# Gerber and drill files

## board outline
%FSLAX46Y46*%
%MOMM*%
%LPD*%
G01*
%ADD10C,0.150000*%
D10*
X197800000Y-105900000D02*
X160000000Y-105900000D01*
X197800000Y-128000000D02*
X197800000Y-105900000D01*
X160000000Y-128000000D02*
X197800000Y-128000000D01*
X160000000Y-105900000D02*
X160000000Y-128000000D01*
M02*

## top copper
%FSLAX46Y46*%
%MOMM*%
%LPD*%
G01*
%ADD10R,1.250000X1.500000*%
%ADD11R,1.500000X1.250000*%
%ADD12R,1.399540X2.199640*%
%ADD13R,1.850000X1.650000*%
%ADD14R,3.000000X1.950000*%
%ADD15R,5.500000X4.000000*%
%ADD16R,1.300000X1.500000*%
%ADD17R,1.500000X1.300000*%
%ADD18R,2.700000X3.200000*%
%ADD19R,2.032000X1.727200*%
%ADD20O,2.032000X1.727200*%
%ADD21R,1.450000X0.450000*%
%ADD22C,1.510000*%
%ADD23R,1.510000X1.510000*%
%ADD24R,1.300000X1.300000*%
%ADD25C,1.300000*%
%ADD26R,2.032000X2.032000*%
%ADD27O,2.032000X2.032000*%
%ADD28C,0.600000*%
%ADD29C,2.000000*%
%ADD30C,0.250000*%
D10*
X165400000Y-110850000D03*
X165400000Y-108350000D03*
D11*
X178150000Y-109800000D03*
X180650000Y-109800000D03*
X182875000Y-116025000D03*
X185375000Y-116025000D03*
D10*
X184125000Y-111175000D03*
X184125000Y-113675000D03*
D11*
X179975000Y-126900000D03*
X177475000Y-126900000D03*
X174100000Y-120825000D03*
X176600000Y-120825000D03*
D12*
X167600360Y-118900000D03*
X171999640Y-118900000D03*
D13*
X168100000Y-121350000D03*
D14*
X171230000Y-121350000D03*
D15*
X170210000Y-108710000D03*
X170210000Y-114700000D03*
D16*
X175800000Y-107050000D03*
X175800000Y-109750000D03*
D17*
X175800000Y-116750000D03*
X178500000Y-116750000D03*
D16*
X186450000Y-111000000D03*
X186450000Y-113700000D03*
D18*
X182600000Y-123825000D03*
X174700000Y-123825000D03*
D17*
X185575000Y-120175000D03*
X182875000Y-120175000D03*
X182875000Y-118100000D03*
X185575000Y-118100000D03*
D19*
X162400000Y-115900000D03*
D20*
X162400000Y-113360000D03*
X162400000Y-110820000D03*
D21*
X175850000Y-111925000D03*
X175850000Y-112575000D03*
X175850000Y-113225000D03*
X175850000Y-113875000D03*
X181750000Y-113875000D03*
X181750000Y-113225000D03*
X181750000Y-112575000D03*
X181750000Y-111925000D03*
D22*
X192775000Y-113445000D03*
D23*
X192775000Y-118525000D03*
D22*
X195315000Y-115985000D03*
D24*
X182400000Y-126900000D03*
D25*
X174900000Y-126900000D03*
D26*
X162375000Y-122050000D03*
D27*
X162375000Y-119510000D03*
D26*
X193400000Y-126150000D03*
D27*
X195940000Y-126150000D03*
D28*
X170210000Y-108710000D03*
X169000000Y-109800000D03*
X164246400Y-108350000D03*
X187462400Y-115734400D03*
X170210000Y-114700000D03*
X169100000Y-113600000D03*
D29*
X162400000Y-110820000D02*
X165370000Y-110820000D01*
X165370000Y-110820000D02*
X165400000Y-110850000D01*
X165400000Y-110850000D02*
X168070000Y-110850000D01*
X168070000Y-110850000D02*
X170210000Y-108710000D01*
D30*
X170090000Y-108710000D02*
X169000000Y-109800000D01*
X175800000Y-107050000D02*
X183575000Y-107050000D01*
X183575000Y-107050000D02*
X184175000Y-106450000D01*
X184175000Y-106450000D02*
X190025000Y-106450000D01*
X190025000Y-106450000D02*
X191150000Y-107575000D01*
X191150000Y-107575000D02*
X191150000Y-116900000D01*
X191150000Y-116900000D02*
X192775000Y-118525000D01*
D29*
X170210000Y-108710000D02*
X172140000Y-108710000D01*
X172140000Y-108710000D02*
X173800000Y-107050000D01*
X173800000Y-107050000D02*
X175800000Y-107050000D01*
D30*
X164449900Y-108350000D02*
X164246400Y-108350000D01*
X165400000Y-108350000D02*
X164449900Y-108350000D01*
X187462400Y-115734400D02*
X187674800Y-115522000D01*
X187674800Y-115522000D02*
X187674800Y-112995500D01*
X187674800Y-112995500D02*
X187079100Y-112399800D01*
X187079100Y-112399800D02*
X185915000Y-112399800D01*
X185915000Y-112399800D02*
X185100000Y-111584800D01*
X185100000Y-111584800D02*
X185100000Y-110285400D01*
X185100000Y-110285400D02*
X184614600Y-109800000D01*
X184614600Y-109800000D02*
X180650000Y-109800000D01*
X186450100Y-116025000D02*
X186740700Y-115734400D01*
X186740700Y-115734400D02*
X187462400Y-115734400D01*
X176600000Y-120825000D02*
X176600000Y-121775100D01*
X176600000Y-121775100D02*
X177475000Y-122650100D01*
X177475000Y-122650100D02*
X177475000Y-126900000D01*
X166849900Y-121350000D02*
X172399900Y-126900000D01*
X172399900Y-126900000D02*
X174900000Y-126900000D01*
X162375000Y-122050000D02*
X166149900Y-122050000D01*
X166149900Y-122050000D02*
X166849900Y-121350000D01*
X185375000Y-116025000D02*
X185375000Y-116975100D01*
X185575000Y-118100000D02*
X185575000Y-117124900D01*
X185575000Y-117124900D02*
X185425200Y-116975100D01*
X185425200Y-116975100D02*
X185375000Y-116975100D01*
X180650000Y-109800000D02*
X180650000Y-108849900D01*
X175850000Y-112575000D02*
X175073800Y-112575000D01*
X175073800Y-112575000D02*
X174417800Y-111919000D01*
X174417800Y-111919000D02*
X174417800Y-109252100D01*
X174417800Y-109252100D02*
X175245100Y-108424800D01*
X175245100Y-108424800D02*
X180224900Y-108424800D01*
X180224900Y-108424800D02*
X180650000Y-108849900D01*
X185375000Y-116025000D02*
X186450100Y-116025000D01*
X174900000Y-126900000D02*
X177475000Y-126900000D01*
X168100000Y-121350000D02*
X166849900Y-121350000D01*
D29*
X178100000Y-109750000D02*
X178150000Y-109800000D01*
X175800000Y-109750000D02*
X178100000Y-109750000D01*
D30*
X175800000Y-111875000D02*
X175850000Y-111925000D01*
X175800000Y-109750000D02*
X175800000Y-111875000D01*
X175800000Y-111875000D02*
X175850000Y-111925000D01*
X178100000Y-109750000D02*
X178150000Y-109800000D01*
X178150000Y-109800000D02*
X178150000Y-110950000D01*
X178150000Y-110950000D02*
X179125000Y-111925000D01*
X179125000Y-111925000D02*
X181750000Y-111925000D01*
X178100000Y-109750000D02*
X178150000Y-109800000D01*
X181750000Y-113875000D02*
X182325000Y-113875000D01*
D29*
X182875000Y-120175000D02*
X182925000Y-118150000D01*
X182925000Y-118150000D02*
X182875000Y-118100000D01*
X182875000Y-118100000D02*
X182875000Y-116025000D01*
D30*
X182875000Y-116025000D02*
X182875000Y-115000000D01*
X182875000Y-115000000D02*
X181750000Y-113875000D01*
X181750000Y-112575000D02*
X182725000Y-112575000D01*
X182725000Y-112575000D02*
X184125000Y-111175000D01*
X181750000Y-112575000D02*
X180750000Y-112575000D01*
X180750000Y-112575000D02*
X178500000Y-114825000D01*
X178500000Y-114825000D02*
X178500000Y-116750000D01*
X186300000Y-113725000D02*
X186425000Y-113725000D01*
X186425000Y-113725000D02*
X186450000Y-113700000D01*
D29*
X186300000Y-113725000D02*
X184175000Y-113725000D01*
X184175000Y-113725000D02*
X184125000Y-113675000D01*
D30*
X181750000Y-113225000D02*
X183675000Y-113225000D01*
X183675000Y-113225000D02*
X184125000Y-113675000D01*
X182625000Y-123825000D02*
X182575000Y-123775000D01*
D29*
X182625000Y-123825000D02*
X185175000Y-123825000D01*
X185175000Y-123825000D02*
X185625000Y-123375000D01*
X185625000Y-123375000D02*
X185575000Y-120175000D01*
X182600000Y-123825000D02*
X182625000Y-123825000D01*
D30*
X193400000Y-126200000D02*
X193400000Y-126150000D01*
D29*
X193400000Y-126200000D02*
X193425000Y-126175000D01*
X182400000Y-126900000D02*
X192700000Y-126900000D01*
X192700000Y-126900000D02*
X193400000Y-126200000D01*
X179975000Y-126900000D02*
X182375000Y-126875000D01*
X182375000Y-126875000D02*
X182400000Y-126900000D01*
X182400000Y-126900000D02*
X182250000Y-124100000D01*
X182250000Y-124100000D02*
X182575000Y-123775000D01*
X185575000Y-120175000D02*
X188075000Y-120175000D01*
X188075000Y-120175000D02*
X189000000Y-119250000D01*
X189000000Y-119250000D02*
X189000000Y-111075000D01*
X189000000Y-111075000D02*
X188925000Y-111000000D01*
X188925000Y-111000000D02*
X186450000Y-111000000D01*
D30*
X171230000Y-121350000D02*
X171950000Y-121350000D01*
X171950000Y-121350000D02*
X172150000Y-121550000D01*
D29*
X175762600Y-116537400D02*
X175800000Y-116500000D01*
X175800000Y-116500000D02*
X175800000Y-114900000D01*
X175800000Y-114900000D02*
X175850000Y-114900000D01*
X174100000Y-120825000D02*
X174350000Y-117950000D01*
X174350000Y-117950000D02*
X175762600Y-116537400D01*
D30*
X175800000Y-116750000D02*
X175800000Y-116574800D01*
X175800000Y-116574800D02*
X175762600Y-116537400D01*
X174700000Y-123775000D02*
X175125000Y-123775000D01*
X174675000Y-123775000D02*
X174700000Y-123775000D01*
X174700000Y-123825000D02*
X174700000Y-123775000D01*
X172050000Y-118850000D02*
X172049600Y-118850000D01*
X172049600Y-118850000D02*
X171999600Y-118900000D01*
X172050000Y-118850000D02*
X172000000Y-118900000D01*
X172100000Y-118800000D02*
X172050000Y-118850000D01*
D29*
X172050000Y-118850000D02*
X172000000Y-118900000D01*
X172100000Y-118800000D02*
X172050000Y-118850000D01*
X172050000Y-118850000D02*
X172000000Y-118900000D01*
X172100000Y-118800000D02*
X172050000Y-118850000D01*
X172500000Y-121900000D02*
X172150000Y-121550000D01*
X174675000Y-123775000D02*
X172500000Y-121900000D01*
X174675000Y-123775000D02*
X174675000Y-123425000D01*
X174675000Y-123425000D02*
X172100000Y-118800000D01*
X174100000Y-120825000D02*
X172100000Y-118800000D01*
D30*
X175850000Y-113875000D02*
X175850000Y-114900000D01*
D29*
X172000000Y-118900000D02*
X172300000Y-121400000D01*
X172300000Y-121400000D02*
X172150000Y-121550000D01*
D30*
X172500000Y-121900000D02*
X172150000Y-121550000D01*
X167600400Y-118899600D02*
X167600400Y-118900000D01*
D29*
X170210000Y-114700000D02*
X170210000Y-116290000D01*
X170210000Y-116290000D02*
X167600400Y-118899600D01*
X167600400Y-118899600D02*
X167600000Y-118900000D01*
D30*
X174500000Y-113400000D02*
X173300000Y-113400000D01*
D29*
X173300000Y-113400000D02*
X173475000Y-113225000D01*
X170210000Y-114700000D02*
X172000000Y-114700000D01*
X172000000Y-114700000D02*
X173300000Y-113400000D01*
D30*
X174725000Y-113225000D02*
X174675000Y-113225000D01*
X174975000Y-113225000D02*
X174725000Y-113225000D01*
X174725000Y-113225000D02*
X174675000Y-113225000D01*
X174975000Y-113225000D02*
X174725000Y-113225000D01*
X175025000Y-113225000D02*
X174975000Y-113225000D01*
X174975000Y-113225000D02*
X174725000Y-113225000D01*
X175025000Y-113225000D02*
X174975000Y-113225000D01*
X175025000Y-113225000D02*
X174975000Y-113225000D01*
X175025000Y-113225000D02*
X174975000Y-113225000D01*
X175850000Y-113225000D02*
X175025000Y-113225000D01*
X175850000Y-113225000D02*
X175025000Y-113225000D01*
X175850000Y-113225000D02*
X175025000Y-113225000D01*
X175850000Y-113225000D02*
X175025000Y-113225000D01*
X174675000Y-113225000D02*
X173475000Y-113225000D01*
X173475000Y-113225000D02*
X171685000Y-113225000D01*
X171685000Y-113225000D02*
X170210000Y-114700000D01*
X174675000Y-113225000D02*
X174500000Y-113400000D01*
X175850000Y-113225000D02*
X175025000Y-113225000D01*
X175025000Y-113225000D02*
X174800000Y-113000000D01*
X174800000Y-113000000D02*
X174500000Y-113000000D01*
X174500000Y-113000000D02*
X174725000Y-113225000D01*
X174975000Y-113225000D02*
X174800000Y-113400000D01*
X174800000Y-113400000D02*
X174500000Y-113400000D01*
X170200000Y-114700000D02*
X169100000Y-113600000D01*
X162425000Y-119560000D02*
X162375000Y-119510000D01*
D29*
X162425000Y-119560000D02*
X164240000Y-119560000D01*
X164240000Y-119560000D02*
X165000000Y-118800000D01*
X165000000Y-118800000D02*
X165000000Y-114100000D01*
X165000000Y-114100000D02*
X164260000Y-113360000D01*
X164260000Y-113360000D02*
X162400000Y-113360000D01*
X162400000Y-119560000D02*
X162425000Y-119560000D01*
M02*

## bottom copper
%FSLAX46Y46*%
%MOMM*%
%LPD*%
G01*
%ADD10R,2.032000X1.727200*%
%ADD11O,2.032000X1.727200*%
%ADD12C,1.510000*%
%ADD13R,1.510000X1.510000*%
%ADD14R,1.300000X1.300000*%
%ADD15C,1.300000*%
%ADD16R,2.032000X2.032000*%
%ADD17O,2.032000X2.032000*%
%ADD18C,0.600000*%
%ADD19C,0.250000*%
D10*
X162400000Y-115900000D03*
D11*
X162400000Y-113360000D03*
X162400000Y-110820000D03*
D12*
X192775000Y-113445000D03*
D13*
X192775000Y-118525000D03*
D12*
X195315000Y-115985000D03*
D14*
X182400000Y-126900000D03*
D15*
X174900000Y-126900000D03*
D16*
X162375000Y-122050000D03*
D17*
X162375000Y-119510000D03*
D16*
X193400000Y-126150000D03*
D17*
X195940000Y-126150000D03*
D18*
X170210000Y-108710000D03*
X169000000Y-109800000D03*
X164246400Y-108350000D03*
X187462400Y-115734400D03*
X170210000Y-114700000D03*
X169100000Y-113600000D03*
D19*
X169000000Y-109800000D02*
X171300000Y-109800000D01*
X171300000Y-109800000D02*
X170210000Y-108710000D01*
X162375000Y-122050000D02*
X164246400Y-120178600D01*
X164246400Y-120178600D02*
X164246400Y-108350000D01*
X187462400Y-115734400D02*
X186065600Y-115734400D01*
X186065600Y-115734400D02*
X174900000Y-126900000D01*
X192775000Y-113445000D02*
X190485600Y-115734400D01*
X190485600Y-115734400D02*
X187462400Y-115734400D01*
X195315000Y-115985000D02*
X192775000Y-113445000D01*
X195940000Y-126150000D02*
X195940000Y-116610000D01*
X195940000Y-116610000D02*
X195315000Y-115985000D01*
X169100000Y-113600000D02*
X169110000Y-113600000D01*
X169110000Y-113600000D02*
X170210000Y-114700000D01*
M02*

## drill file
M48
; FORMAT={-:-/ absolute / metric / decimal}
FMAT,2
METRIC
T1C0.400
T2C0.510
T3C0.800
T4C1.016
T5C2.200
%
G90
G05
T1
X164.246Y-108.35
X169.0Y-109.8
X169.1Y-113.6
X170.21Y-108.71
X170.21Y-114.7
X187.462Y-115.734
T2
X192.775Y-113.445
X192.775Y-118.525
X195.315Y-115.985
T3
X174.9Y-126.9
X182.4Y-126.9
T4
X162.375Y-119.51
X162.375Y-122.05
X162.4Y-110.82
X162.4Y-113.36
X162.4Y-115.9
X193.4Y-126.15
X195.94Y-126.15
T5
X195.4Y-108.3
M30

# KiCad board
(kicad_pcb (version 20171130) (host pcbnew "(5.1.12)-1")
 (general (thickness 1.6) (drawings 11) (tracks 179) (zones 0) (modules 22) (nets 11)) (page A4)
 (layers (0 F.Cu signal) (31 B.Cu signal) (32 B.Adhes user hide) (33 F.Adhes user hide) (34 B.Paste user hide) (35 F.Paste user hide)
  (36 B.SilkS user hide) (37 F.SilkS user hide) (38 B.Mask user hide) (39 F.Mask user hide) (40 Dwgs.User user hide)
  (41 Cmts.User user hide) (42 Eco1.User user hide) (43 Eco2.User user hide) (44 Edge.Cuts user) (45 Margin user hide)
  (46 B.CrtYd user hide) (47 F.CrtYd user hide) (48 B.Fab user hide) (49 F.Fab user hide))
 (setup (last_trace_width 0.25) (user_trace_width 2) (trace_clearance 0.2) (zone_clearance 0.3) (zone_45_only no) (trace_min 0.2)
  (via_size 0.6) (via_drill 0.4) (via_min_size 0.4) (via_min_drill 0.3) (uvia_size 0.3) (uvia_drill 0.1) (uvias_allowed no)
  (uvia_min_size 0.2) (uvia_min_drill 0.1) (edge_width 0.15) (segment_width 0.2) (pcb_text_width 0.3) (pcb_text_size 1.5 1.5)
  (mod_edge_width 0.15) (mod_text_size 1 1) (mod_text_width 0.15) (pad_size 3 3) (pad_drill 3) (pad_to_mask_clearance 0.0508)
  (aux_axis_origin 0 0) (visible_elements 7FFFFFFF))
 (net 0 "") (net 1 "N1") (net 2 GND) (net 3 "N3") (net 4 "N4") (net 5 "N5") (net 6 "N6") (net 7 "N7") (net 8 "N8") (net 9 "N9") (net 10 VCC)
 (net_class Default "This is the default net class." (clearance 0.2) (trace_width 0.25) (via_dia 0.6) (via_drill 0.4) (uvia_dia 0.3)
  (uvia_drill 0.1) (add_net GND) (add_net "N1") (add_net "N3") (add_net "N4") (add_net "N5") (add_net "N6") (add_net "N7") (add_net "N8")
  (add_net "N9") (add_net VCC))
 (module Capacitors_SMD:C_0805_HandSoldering (layer F.Cu) (at 165.4 109.6 90)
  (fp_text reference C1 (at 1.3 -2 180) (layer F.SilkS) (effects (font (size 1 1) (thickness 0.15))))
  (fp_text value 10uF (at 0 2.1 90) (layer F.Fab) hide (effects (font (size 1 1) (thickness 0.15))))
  (pad 1 smd rect (at -1.25 0 90) (size 1.5 1.25) (layers F.Cu F.Paste F.Mask) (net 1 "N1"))
  (pad 2 smd rect (at 1.25 0 90) (size 1.5 1.25) (layers F.Cu F.Paste F.Mask) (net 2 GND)))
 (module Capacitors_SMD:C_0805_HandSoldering (layer F.Cu) (at 179.4 109.8)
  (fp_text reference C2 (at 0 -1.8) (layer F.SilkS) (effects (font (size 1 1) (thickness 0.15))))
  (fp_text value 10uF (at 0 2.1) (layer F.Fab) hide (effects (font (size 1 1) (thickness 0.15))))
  (pad 1 smd rect (at -1.25 0) (size 1.5 1.25) (layers F.Cu F.Paste F.Mask) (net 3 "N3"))
  (pad 2 smd rect (at 1.25 0) (size 1.5 1.25) (layers F.Cu F.Paste F.Mask) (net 2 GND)))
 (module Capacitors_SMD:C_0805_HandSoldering (layer F.Cu) (at 184.125 116.025)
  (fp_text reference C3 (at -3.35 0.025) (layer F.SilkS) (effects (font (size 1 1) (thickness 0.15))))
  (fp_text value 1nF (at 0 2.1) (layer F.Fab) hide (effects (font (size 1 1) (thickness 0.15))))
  (pad 1 smd rect (at -1.25 0) (size 1.5 1.25) (layers F.Cu F.Paste F.Mask) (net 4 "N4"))
  (pad 2 smd rect (at 1.25 0) (size 1.5 1.25) (layers F.Cu F.Paste F.Mask) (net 2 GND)))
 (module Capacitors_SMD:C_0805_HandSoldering (layer F.Cu) (at 184.125 112.425 270)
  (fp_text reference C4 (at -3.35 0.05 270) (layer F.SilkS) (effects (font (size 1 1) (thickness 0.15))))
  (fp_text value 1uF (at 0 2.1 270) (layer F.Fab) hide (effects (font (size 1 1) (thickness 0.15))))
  (pad 1 smd rect (at -1.25 0 270) (size 1.5 1.25) (layers F.Cu F.Paste F.Mask) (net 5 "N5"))
  (pad 2 smd rect (at 1.25 0 270) (size 1.5 1.25) (layers F.Cu F.Paste F.Mask) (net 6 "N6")))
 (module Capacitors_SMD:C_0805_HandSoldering (layer F.Cu) (at 178.725 126.9 180)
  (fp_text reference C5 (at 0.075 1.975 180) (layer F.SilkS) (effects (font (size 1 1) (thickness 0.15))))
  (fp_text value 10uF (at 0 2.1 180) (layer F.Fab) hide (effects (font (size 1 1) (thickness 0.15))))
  (pad 1 smd rect (at -1.25 0 180) (size 1.5 1.25) (layers F.Cu F.Paste F.Mask) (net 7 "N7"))
  (pad 2 smd rect (at 1.25 0 180) (size 1.5 1.25) (layers F.Cu F.Paste F.Mask) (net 2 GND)))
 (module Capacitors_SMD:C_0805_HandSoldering (layer F.Cu) (at 175.35 120.825)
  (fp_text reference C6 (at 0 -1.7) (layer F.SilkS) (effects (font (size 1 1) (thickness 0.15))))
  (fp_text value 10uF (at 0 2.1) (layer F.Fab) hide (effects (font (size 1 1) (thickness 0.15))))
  (pad 1 smd rect (at -1.25 0) (size 1.5 1.25) (layers F.Cu F.Paste F.Mask) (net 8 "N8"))
  (pad 2 smd rect (at 1.25 0) (size 1.5 1.25) (layers F.Cu F.Paste F.Mask) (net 2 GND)))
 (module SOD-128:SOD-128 (layer F.Cu) (at 169.8 118.9)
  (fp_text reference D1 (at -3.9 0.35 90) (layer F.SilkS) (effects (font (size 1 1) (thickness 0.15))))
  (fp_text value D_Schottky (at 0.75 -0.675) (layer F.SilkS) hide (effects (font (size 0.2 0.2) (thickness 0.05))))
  (pad 2 smd rect (at -2.19964 0) (size 1.39954 2.19964) (layers F.Cu F.Paste F.Mask) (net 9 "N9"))
  (pad 1 smd rect (at 2.19964 0) (size 1.39954 2.19964) (layers F.Cu F.Paste F.Mask) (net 8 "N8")))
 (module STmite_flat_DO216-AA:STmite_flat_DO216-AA (layer F.Cu) (at 168.55 120.4)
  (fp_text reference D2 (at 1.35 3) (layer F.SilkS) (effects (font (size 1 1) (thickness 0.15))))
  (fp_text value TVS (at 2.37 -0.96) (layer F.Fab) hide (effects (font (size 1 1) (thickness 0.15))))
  (pad 1 smd rect (at -0.45 0.95) (size 1.85 1.65) (layers F.Cu F.Paste F.Mask) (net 2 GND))
  (pad 2 smd rect (at 2.68 0.95) (size 3 1.95) (layers F.Cu F.Paste F.Mask) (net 8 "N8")))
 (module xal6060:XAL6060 (layer F.Cu) (at 166.9 114.9 90)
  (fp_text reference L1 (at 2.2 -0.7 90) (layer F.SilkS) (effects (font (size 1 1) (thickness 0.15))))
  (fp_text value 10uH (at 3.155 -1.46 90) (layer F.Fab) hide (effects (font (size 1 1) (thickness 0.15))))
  (pad 2 smd rect (at 6.19 3.31 90) (size 4 5.5) (layers F.Cu F.Paste F.Mask) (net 1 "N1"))
  (pad 1 smd rect (at 0.2 3.31 90) (size 4 5.5) (layers F.Cu F.Paste F.Mask) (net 9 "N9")))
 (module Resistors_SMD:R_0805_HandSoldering (layer F.Cu) (at 175.8 108.4 270)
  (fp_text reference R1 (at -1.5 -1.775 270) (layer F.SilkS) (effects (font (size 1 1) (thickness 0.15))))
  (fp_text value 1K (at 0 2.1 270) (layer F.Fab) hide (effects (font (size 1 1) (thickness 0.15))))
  (pad 1 smd rect (at -1.35 0 270) (size 1.5 1.3) (layers F.Cu F.Paste F.Mask) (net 1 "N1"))
  (pad 2 smd rect (at 1.35 0 270) (size 1.5 1.3) (layers F.Cu F.Paste F.Mask) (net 3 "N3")))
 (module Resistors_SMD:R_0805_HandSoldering (layer F.Cu) (at 177.15 116.75)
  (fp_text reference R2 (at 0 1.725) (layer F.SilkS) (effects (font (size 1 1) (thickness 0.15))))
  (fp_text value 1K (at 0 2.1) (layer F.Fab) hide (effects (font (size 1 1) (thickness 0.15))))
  (pad 1 smd rect (at -1.35 0) (size 1.5 1.3) (layers F.Cu F.Paste F.Mask) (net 8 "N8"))
  (pad 2 smd rect (at 1.35 0) (size 1.5 1.3) (layers F.Cu F.Paste F.Mask) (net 5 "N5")))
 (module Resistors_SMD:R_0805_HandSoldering (layer F.Cu) (at 186.45 112.35 270)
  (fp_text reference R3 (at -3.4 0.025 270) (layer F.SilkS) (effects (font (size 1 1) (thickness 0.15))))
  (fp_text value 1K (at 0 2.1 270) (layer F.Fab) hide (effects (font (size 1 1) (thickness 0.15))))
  (pad 1 smd rect (at -1.35 0 270) (size 1.5 1.3) (layers F.Cu F.Paste F.Mask) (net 7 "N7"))
  (pad 2 smd rect (at 1.35 0 270) (size 1.5 1.3) (layers F.Cu F.Paste F.Mask) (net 6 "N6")))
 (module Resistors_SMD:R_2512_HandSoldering (layer F.Cu) (at 178.65 123.825 180)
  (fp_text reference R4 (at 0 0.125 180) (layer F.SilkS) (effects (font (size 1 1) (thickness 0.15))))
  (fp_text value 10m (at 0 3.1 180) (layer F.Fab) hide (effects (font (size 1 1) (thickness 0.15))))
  (pad 1 smd rect (at -3.95 0 180) (size 2.7 3.2) (layers F.Cu F.Paste F.Mask) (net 7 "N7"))
  (pad 2 smd rect (at 3.95 0 180) (size 2.7 3.2) (layers F.Cu F.Paste F.Mask) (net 8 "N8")))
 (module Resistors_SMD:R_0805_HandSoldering (layer F.Cu) (at 184.225 120.175 180)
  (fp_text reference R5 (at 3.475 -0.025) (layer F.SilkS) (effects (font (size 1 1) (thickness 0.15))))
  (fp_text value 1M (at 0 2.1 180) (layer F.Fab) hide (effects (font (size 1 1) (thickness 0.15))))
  (pad 1 smd rect (at -1.35 0 180) (size 1.5 1.3) (layers F.Cu F.Paste F.Mask) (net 7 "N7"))
  (pad 2 smd rect (at 1.35 0 180) (size 1.5 1.3) (layers F.Cu F.Paste F.Mask) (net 4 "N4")))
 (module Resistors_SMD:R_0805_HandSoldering (layer F.Cu) (at 184.225 118.1)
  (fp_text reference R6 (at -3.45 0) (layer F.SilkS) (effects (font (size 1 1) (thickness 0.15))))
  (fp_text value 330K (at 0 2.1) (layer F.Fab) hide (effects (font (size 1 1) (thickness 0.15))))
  (pad 1 smd rect (at -1.35 0) (size 1.5 1.3) (layers F.Cu F.Paste F.Mask) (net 4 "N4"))
  (pad 2 smd rect (at 1.35 0) (size 1.5 1.3) (layers F.Cu F.Paste F.Mask) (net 2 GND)))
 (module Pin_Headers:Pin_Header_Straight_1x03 (layer F.Cu) (at 162.4 115.9 180)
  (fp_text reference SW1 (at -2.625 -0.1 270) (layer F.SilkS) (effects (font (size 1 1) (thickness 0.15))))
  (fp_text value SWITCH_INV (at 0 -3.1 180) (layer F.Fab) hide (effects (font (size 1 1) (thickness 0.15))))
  (pad 1 thru_hole rect (at 0 0 180) (size 2.032 1.7272) (drill 1.016) (layers *.Cu *.Mask F.SilkS))
  (pad 2 thru_hole oval (at 0 2.54 180) (size 2.032 1.7272) (drill 1.016) (layers *.Cu *.Mask F.SilkS) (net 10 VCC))
  (pad 3 thru_hole oval (at 0 5.08 180) (size 2.032 1.7272) (drill 1.016) (layers *.Cu *.Mask F.SilkS) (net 1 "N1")))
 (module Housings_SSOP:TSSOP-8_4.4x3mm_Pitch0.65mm (layer F.Cu) (at 178.8 112.9)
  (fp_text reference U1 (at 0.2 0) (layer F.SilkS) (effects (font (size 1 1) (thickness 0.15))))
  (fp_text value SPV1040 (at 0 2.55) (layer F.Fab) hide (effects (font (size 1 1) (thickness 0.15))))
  (pad 1 smd rect (at -2.95 -0.975) (size 1.45 0.45) (layers F.Cu F.Paste F.Mask) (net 3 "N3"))
  (pad 2 smd rect (at -2.95 -0.325) (size 1.45 0.45) (layers F.Cu F.Paste F.Mask) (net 2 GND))
  (pad 3 smd rect (at -2.95 0.325) (size 1.45 0.45) (layers F.Cu F.Paste F.Mask) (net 9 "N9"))
  (pad 4 smd rect (at -2.95 0.975) (size 1.45 0.45) (layers F.Cu F.Paste F.Mask) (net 8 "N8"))
  (pad 5 smd rect (at 2.95 0.975) (size 1.45 0.45) (layers F.Cu F.Paste F.Mask) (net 4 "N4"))
  (pad 6 smd rect (at 2.95 0.325) (size 1.45 0.45) (layers F.Cu F.Paste F.Mask) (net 6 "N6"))
  (pad 7 smd rect (at 2.95 -0.325) (size 1.45 0.45) (layers F.Cu F.Paste F.Mask) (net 5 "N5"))
  (pad 8 smd rect (at 2.95 -0.975) (size 1.45 0.45) (layers F.Cu F.Paste F.Mask) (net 3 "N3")))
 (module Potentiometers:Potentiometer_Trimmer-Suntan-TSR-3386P (layer F.Cu) (at 192.775 118.525 90)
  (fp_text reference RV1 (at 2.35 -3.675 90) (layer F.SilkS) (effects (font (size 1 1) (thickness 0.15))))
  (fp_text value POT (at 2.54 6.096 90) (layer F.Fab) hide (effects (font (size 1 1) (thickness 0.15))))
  (pad 3 thru_hole circle (at 5.08 0 90) (size 1.51 1.51) (drill 0.51) (layers *.Cu *.Mask F.SilkS) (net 2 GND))
  (pad 1 thru_hole rect (at 0 0 90) (size 1.51 1.51) (drill 0.51) (layers *.Cu *.Mask F.SilkS) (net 1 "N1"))
  (pad 2 thru_hole circle (at 2.54 2.54 90) (size 1.51 1.51) (drill 0.51) (layers *.Cu *.Mask F.SilkS) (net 2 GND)))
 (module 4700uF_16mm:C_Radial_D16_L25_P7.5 (layer F.Cu) (at 182.4 126.9 180)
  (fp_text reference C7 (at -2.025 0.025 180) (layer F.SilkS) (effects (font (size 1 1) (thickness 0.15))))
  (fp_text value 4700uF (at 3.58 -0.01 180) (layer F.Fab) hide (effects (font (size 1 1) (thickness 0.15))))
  (pad 1 thru_hole rect (at 0 0 180) (size 1.3 1.3) (drill 0.8) (layers *.Cu *.Mask F.SilkS) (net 7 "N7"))
  (pad 2 thru_hole circle (at 7.5 0 180) (size 1.3 1.3) (drill 0.8) (layers *.Cu *.Mask F.SilkS) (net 2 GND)))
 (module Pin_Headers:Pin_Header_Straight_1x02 (layer F.Cu) (at 162.375 122.05 180)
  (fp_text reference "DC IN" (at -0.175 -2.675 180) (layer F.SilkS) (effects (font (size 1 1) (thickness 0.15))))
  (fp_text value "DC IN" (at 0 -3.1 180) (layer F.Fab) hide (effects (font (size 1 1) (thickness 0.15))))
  (pad 1 thru_hole rect (at 0 0 180) (size 2.032 2.032) (drill 1.016) (layers *.Cu *.Mask F.SilkS) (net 2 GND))
  (pad 2 thru_hole oval (at 0 2.54 180) (size 2.032 2.032) (drill 1.016) (layers *.Cu *.Mask F.SilkS) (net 10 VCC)))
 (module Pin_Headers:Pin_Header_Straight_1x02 (layer F.Cu) (at 193.4 126.15 90)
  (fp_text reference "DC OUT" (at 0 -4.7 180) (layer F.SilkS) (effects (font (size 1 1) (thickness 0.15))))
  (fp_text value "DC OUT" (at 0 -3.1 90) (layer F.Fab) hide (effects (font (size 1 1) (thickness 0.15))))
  (pad 1 thru_hole rect (at 0 0 90) (size 2.032 2.032) (drill 1.016) (layers *.Cu *.Mask F.SilkS) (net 7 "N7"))
  (pad 2 thru_hole oval (at 0 2.54 90) (size 2.032 2.032) (drill 1.016) (layers *.Cu *.Mask F.SilkS) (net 2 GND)))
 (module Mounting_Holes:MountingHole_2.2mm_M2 (layer F.Cu) (at 195.4 108.3)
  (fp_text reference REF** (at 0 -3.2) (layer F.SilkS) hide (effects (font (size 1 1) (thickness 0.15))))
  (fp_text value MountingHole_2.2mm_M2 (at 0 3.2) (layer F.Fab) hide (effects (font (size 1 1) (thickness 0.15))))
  (pad 1 np_thru_hole circle (at 0 0) (size 2.2 2.2) (drill 2.2) (layers *.Cu *.Mask F.SilkS)))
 (gr_line (start 197.8 105.9) (end 160 105.9) (angle 90) (layer Edge.Cuts) (width 0.15))
 (gr_line (start 197.8 128) (end 197.8 105.9) (angle 90) (layer Edge.Cuts) (width 0.15))
 (gr_line (start 160 128) (end 197.8 128) (angle 90) (layer Edge.Cuts) (width 0.15))
 (gr_line (start 160 105.9) (end 160 128) (angle 90) (layer Edge.Cuts) (width 0.15))
 (segment (start 162.4 110.82) (end 165.37 110.82) (width 2) (layer F.Cu) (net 1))
 (segment (start 165.37 110.82) (end 165.4 110.85) (width 2) (layer F.Cu) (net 1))
 (segment (start 165.4 110.85) (end 168.07 110.85) (width 2) (layer F.Cu) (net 1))
 (segment (start 168.07 110.85) (end 170.21 108.71) (width 2) (layer F.Cu) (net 1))
 (segment (start 169 109.8) (end 171.3 109.8) (width 0.25) (layer B.Cu) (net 1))
 (segment (start 171.3 109.8) (end 170.21 108.71) (width 0.25) (layer B.Cu) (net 1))
 (segment (start 170.09 108.71) (end 169 109.8) (width 0.25) (layer F.Cu) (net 1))
 (segment (start 175.8 107.05) (end 183.575 107.05) (width 0.25) (layer F.Cu) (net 1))
 (segment (start 183.575 107.05) (end 184.175 106.45) (width 0.25) (layer F.Cu) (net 1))
 (segment (start 184.175 106.45) (end 190.025 106.45) (width 0.25) (layer F.Cu) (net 1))
 (segment (start 190.025 106.45) (end 191.15 107.575) (width 0.25) (layer F.Cu) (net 1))
 (segment (start 191.15 107.575) (end 191.15 116.9) (width 0.25) (layer F.Cu) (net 1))
 (segment (start 191.15 116.9) (end 192.775 118.525) (width 0.25) (layer F.Cu) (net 1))
 (segment (start 170.21 108.71) (end 172.14 108.71) (width 2) (layer F.Cu) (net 1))
 (segment (start 172.14 108.71) (end 173.8 107.05) (width 2) (layer F.Cu) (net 1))
 (segment (start 173.8 107.05) (end 175.8 107.05) (width 2) (layer F.Cu) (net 1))
 (via (at 170.21 108.71) (size 0.6) (layers F.Cu B.Cu) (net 1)) (via (at 169 109.8) (size 0.6) (layers F.Cu B.Cu) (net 1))
 (segment (start 164.4499 108.35) (end 164.2464 108.35) (width 0.25) (layer F.Cu) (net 2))
 (segment (start 162.375 122.05) (end 164.2464 120.1786) (width 0.25) (layer B.Cu) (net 2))
 (segment (start 164.2464 120.1786) (end 164.2464 108.35) (width 0.25) (layer B.Cu) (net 2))
 (segment (start 165.4 108.35) (end 164.4499 108.35) (width 0.25) (layer F.Cu) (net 2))
 (segment (start 187.4624 115.7344) (end 186.0656 115.7344) (width 0.25) (layer B.Cu) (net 2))
 (segment (start 186.0656 115.7344) (end 174.9 126.9) (width 0.25) (layer B.Cu) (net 2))
 (segment (start 192.775 113.445) (end 190.4856 115.7344) (width 0.25) (layer B.Cu) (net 2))
 (segment (start 190.4856 115.7344) (end 187.4624 115.7344) (width 0.25) (layer B.Cu) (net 2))
 (segment (start 187.4624 115.7344) (end 187.6748 115.522) (width 0.25) (layer F.Cu) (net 2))
 (segment (start 187.6748 115.522) (end 187.6748 112.9955) (width 0.25) (layer F.Cu) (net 2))
 (segment (start 187.6748 112.9955) (end 187.0791 112.3998) (width 0.25) (layer F.Cu) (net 2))
 (segment (start 187.0791 112.3998) (end 185.915 112.3998) (width 0.25) (layer F.Cu) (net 2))
 (segment (start 185.915 112.3998) (end 185.1 111.5848) (width 0.25) (layer F.Cu) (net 2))
 (segment (start 185.1 111.5848) (end 185.1 110.2854) (width 0.25) (layer F.Cu) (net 2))
 (segment (start 185.1 110.2854) (end 184.6146 109.8) (width 0.25) (layer F.Cu) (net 2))
 (segment (start 184.6146 109.8) (end 180.65 109.8) (width 0.25) (layer F.Cu) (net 2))
 (segment (start 186.4501 116.025) (end 186.7407 115.7344) (width 0.25) (layer F.Cu) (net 2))
 (segment (start 186.7407 115.7344) (end 187.4624 115.7344) (width 0.25) (layer F.Cu) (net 2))
 (segment (start 176.6 120.825) (end 176.6 121.7751) (width 0.25) (layer F.Cu) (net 2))
 (segment (start 176.6 121.7751) (end 177.475 122.6501) (width 0.25) (layer F.Cu) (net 2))
 (segment (start 177.475 122.6501) (end 177.475 126.9) (width 0.25) (layer F.Cu) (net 2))
 (segment (start 166.8499 121.35) (end 172.3999 126.9) (width 0.25) (layer F.Cu) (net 2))
 (segment (start 172.3999 126.9) (end 174.9 126.9) (width 0.25) (layer F.Cu) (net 2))
 (segment (start 162.375 122.05) (end 166.1499 122.05) (width 0.25) (layer F.Cu) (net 2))
 (segment (start 166.1499 122.05) (end 166.8499 121.35) (width 0.25) (layer F.Cu) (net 2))
 (segment (start 185.375 116.025) (end 185.375 116.9751) (width 0.25) (layer F.Cu) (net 2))
 (segment (start 185.575 118.1) (end 185.575 117.1249) (width 0.25) (layer F.Cu) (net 2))
 (segment (start 185.575 117.1249) (end 185.4252 116.9751) (width 0.25) (layer F.Cu) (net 2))
 (segment (start 185.4252 116.9751) (end 185.375 116.9751) (width 0.25) (layer F.Cu) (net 2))
 (segment (start 180.65 109.8) (end 180.65 108.8499) (width 0.25) (layer F.Cu) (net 2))
 (segment (start 175.85 112.575) (end 175.0738 112.575) (width 0.25) (layer F.Cu) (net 2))
 (segment (start 175.0738 112.575) (end 174.4178 111.919) (width 0.25) (layer F.Cu) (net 2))
 (segment (start 174.4178 111.919) (end 174.4178 109.2521) (width 0.25) (layer F.Cu) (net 2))
 (segment (start 174.4178 109.2521) (end 175.2451 108.4248) (width 0.25) (layer F.Cu) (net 2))
 (segment (start 175.2451 108.4248) (end 180.2249 108.4248) (width 0.25) (layer F.Cu) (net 2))
 (segment (start 180.2249 108.4248) (end 180.65 108.8499) (width 0.25) (layer F.Cu) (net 2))
 (segment (start 185.375 116.025) (end 186.4501 116.025) (width 0.25) (layer F.Cu) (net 2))
 (segment (start 195.315 115.985) (end 192.775 113.445) (width 0.25) (layer B.Cu) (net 2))
 (segment (start 195.94 126.15) (end 195.94 116.61) (width 0.25) (layer B.Cu) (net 2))
 (segment (start 195.94 116.61) (end 195.315 115.985) (width 0.25) (layer B.Cu) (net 2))
 (segment (start 174.9 126.9) (end 177.475 126.9) (width 0.25) (layer F.Cu) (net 2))
 (segment (start 168.1 121.35) (end 166.8499 121.35) (width 0.25) (layer F.Cu) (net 2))
 (via (at 164.2464 108.35) (size 0.6) (layers F.Cu B.Cu) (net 2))
 (via (at 187.4624 115.7344) (size 0.6) (layers F.Cu B.Cu) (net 2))
 (segment (start 178.1 109.75) (end 178.15 109.8) (width 2) (layer F.Cu) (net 3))
 (segment (start 175.8 109.75) (end 178.1 109.75) (width 2) (layer F.Cu) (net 3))
 (segment (start 175.8 111.875) (end 175.85 111.925) (width 0.25) (layer F.Cu) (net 3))
 (segment (start 175.8 109.75) (end 175.8 111.875) (width 0.25) (layer F.Cu) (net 3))
 (segment (start 175.8 111.875) (end 175.85 111.925) (width 0.25) (layer F.Cu) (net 3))
 (segment (start 178.1 109.75) (end 178.15 109.8) (width 0.25) (layer F.Cu) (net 3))
 (segment (start 178.15 109.8) (end 178.15 110.95) (width 0.25) (layer F.Cu) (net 3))
 (segment (start 178.15 110.95) (end 179.125 111.925) (width 0.25) (layer F.Cu) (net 3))
 (segment (start 179.125 111.925) (end 181.75 111.925) (width 0.25) (layer F.Cu) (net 3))
 (segment (start 178.1 109.75) (end 178.15 109.8) (width 0.25) (layer F.Cu) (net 3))
 (segment (start 181.75 113.875) (end 182.325 113.875) (width 0.25) (layer F.Cu) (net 4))
 (segment (start 182.875 120.175) (end 182.925 118.15) (width 2) (layer F.Cu) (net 4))
 (segment (start 182.925 118.15) (end 182.875 118.1) (width 2) (layer F.Cu) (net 4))
 (segment (start 182.875 118.1) (end 182.875 116.025) (width 2) (layer F.Cu) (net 4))
 (segment (start 182.875 116.025) (end 182.875 115) (width 0.25) (layer F.Cu) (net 4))
 (segment (start 182.875 115) (end 181.75 113.875) (width 0.25) (layer F.Cu) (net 4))
 (segment (start 181.75 112.575) (end 182.725 112.575) (width 0.25) (layer F.Cu) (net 5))
 (segment (start 182.725 112.575) (end 184.125 111.175) (width 0.25) (layer F.Cu) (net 5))
 (segment (start 181.75 112.575) (end 180.75 112.575) (width 0.25) (layer F.Cu) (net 5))
 (segment (start 180.75 112.575) (end 178.5 114.825) (width 0.25) (layer F.Cu) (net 5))
 (segment (start 178.5 114.825) (end 178.5 116.75) (width 0.25) (layer F.Cu) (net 5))
 (segment (start 186.3 113.725) (end 186.425 113.725) (width 0.25) (layer F.Cu) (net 6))
 (segment (start 186.425 113.725) (end 186.45 113.7) (width 0.25) (layer F.Cu) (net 6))
 (segment (start 186.3 113.725) (end 184.175 113.725) (width 2) (layer F.Cu) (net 6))
 (segment (start 184.175 113.725) (end 184.125 113.675) (width 2) (layer F.Cu) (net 6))
 (segment (start 181.75 113.225) (end 183.675 113.225) (width 0.25) (layer F.Cu) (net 6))
 (segment (start 183.675 113.225) (end 184.125 113.675) (width 0.25) (layer F.Cu) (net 6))
 (segment (start 182.625 123.825) (end 182.575 123.775) (width 0.25) (layer F.Cu) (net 7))
 (segment (start 182.625 123.825) (end 185.175 123.825) (width 2) (layer F.Cu) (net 7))
 (segment (start 185.175 123.825) (end 185.625 123.375) (width 2) (layer F.Cu) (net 7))
 (segment (start 185.625 123.375) (end 185.575 120.175) (width 2) (layer F.Cu) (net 7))
 (segment (start 182.6 123.825) (end 182.625 123.825) (width 2) (layer F.Cu) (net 7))
 (segment (start 193.4 126.2) (end 193.4 126.15) (width 0.25) (layer F.Cu) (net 7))
 (segment (start 193.4 126.2) (end 193.425 126.175) (width 2) (layer F.Cu) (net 7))
 (segment (start 182.4 126.9) (end 192.7 126.9) (width 2) (layer F.Cu) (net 7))
 (segment (start 192.7 126.9) (end 193.4 126.2) (width 2) (layer F.Cu) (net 7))
 (segment (start 179.975 126.9) (end 182.375 126.875) (width 2) (layer F.Cu) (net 7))
 (segment (start 182.375 126.875) (end 182.4 126.9) (width 2) (layer F.Cu) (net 7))
 (segment (start 182.4 126.9) (end 182.25 124.1) (width 2) (layer F.Cu) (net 7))
 (segment (start 182.25 124.1) (end 182.575 123.775) (width 2) (layer F.Cu) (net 7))
 (segment (start 185.575 120.175) (end 188.075 120.175) (width 2) (layer F.Cu) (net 7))
 (segment (start 188.075 120.175) (end 189 119.25) (width 2) (layer F.Cu) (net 7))
 (segment (start 189 119.25) (end 189 111.075) (width 2) (layer F.Cu) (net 7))
 (segment (start 189 111.075) (end 188.925 111) (width 2) (layer F.Cu) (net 7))
 (segment (start 188.925 111) (end 186.45 111) (width 2) (layer F.Cu) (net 7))
 (segment (start 171.23 121.35) (end 171.95 121.35) (width 0.25) (layer F.Cu) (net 8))
 (segment (start 171.95 121.35) (end 172.15 121.55) (width 0.25) (layer F.Cu) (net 8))
 (segment (start 175.7626 116.5374) (end 175.8 116.5) (width 2) (layer F.Cu) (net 8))
 (segment (start 175.8 116.5) (end 175.8 114.9) (width 2) (layer F.Cu) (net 8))
 (segment (start 175.8 114.9) (end 175.85 114.9) (width 2) (layer F.Cu) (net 8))
 (segment (start 174.1 120.825) (end 174.35 117.95) (width 2) (layer F.Cu) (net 8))
 (segment (start 174.35 117.95) (end 175.7626 116.5374) (width 2) (layer F.Cu) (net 8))
 (segment (start 175.8 116.75) (end 175.8 116.5748) (width 0.25) (layer F.Cu) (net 8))
 (segment (start 175.8 116.5748) (end 175.7626 116.5374) (width 0.25) (layer F.Cu) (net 8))
 (segment (start 174.7 123.775) (end 175.125 123.775) (width 0.25) (layer F.Cu) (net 8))
 (segment (start 174.675 123.775) (end 174.7 123.775) (width 0.25) (layer F.Cu) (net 8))
 (segment (start 174.7 123.825) (end 174.7 123.775) (width 0.25) (layer F.Cu) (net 8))
 (segment (start 172.05 118.85) (end 172.0496 118.85) (width 0.25) (layer F.Cu) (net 8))
 (segment (start 172.0496 118.85) (end 171.9996 118.9) (width 0.25) (layer F.Cu) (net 8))
 (segment (start 172.05 118.85) (end 172 118.9) (width 0.25) (layer F.Cu) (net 8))
 (segment (start 172.1 118.8) (end 172.05 118.85) (width 0.25) (layer F.Cu) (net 8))
 (segment (start 172.05 118.85) (end 172 118.9) (width 2) (layer F.Cu) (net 8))
 (segment (start 172.1 118.8) (end 172.05 118.85) (width 2) (layer F.Cu) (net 8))
 (segment (start 172.05 118.85) (end 172 118.9) (width 2) (layer F.Cu) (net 8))
 (segment (start 172.1 118.8) (end 172.05 118.85) (width 2) (layer F.Cu) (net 8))
 (segment (start 172.5 121.9) (end 172.15 121.55) (width 2) (layer F.Cu) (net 8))
 (segment (start 174.675 123.775) (end 172.5 121.9) (width 2) (layer F.Cu) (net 8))
 (segment (start 174.675 123.775) (end 174.675 123.425) (width 2) (layer F.Cu) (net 8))
 (segment (start 174.675 123.425) (end 172.1 118.8) (width 2) (layer F.Cu) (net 8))
 (segment (start 174.1 120.825) (end 172.1 118.8) (width 2) (layer F.Cu) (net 8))
 (segment (start 175.85 113.875) (end 175.85 114.9) (width 0.25) (layer F.Cu) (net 8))
 (segment (start 172 118.9) (end 172.3 121.4) (width 2) (layer F.Cu) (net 8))
 (segment (start 172.3 121.4) (end 172.15 121.55) (width 2) (layer F.Cu) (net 8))
 (segment (start 172.5 121.9) (end 172.15 121.55) (width 0.25) (layer F.Cu) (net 8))
 (segment (start 167.6004 118.8996) (end 167.6004 118.9) (width 0.25) (layer F.Cu) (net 9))
 (segment (start 170.21 114.7) (end 170.21 116.29) (width 2) (layer F.Cu) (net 9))
 (segment (start 170.21 116.29) (end 167.6004 118.8996) (width 2) (layer F.Cu) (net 9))
 (segment (start 167.6004 118.8996) (end 167.6 118.9) (width 2) (layer F.Cu) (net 9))
 (segment (start 174.5 113.4) (end 173.3 113.4) (width 0.25) (layer F.Cu) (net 9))
 (segment (start 173.3 113.4) (end 173.475 113.225) (width 2) (layer F.Cu) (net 9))
 (segment (start 170.21 114.7) (end 172 114.7) (width 2) (layer F.Cu) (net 9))
 (segment (start 172 114.7) (end 173.3 113.4) (width 2) (layer F.Cu) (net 9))
 (segment (start 174.725 113.225) (end 174.675 113.225) (width 0.25) (layer F.Cu) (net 9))
 (segment (start 174.975 113.225) (end 174.725 113.225) (width 0.25) (layer F.Cu) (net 9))
 (segment (start 174.725 113.225) (end 174.675 113.225) (width 0.25) (layer F.Cu) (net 9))
 (segment (start 174.975 113.225) (end 174.725 113.225) (width 0.25) (layer F.Cu) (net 9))
 (segment (start 175.025 113.225) (end 174.975 113.225) (width 0.25) (layer F.Cu) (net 9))
 (segment (start 174.975 113.225) (end 174.725 113.225) (width 0.25) (layer F.Cu) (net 9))
 (segment (start 175.025 113.225) (end 174.975 113.225) (width 0.25) (layer F.Cu) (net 9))
 (segment (start 175.025 113.225) (end 174.975 113.225) (width 0.25) (layer F.Cu) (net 9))
 (segment (start 175.025 113.225) (end 174.975 113.225) (width 0.25) (layer F.Cu) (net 9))
 (segment (start 175.85 113.225) (end 175.025 113.225) (width 0.25) (layer F.Cu) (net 9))
 (segment (start 175.85 113.225) (end 175.025 113.225) (width 0.25) (layer F.Cu) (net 9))
 (segment (start 175.85 113.225) (end 175.025 113.225) (width 0.25) (layer F.Cu) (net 9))
 (segment (start 175.85 113.225) (end 175.025 113.225) (width 0.25) (layer F.Cu) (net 9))
 (segment (start 174.675 113.225) (end 173.475 113.225) (width 0.25) (layer F.Cu) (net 9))
 (segment (start 173.475 113.225) (end 171.685 113.225) (width 0.25) (layer F.Cu) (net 9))
 (segment (start 171.685 113.225) (end 170.21 114.7) (width 0.25) (layer F.Cu) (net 9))
 (segment (start 174.675 113.225) (end 174.5 113.4) (width 0.25) (layer F.Cu) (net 9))
 (segment (start 175.85 113.225) (end 175.025 113.225) (width 0.25) (layer F.Cu) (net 9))
 (segment (start 175.025 113.225) (end 174.8 113) (width 0.25) (layer F.Cu) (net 9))
 (segment (start 174.8 113) (end 174.5 113) (width 0.25) (layer F.Cu) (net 9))
 (segment (start 174.5 113) (end 174.725 113.225) (width 0.25) (layer F.Cu) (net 9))
 (segment (start 174.975 113.225) (end 174.8 113.4) (width 0.25) (layer F.Cu) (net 9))
 (segment (start 174.8 113.4) (end 174.5 113.4) (width 0.25) (layer F.Cu) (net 9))
 (segment (start 169.1 113.6) (end 169.11 113.6) (width 0.25) (layer B.Cu) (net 9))
 (segment (start 169.11 113.6) (end 170.21 114.7) (width 0.25) (layer B.Cu) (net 9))
 (segment (start 170.2 114.7) (end 169.1 113.6) (width 0.25) (layer F.Cu) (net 9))
 (via (at 170.21 114.7) (size 0.6) (layers F.Cu B.Cu) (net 9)) (via (at 169.1 113.6) (size 0.6) (layers F.Cu B.Cu) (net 9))
 (segment (start 162.425 119.56) (end 162.375 119.51) (width 0.25) (layer F.Cu) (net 10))
 (segment (start 162.425 119.56) (end 164.24 119.56) (width 2) (layer F.Cu) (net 10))
 (segment (start 164.24 119.56) (end 165 118.8) (width 2) (layer F.Cu) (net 10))
 (segment (start 165 118.8) (end 165 114.1) (width 2) (layer F.Cu) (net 10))
 (segment (start 165 114.1) (end 164.26 113.36) (width 2) (layer F.Cu) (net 10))
 (segment (start 164.26 113.36) (end 162.4 113.36) (width 2) (layer F.Cu) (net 10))
 (segment (start 162.4 119.56) (end 162.425 119.56) (width 2) (layer F.Cu) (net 10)))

